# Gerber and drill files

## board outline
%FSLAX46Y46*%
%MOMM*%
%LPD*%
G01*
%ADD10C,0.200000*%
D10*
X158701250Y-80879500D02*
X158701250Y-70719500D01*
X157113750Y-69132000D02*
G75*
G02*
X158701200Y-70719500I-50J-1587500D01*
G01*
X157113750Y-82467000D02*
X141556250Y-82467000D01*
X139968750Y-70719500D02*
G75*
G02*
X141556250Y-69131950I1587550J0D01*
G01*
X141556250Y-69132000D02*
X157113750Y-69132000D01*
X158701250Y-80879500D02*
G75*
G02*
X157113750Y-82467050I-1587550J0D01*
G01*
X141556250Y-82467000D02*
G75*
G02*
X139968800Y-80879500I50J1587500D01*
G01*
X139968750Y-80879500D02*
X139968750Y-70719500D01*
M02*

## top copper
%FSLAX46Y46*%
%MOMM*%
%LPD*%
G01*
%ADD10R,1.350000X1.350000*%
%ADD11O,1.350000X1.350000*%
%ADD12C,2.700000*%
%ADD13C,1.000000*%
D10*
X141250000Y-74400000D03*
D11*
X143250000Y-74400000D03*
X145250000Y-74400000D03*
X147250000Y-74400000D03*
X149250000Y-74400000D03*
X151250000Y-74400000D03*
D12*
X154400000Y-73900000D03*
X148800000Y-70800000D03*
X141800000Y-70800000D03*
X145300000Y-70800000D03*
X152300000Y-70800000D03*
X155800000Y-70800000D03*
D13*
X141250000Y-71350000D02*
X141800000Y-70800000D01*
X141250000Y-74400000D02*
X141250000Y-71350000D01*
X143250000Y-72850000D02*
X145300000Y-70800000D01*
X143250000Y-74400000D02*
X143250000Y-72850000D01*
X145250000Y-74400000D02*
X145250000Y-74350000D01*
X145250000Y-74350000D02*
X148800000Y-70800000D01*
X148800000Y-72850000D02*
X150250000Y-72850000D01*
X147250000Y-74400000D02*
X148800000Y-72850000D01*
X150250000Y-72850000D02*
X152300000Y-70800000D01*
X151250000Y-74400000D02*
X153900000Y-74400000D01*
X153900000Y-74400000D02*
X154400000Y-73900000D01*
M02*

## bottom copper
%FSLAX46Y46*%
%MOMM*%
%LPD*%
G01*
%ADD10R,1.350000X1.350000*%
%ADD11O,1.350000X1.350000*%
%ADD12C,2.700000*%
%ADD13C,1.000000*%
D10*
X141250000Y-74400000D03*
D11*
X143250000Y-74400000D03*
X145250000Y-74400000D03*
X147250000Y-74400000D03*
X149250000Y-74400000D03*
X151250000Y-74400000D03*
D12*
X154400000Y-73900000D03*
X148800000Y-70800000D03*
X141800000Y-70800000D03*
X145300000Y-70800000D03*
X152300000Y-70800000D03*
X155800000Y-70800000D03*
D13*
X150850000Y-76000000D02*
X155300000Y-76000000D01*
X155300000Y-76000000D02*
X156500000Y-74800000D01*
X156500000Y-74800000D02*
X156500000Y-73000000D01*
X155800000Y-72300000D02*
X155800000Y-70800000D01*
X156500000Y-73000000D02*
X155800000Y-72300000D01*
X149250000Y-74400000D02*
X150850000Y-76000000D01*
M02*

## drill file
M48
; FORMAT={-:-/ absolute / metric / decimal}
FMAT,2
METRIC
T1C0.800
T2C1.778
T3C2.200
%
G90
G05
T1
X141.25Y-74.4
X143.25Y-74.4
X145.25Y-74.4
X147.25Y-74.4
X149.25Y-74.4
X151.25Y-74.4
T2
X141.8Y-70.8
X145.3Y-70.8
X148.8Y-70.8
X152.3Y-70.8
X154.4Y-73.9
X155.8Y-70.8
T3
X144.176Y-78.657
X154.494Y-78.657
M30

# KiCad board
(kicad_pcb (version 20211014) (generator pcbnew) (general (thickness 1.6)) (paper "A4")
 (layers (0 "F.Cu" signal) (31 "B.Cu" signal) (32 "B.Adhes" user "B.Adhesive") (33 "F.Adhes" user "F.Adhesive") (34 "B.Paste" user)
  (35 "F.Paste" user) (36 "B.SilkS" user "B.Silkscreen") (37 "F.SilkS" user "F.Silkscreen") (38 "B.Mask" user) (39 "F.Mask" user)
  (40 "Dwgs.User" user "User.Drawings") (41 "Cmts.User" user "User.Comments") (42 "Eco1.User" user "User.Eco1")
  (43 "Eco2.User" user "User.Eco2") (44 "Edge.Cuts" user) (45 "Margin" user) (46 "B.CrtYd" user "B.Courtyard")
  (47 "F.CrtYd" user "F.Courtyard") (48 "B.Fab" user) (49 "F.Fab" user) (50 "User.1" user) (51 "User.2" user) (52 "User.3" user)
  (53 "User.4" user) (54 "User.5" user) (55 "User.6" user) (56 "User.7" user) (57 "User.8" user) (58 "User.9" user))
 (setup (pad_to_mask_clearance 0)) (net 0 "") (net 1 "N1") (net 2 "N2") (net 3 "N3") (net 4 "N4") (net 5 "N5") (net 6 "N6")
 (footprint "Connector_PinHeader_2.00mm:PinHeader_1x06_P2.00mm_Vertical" (layer "F.Cu") (at 141.25 74.4 90)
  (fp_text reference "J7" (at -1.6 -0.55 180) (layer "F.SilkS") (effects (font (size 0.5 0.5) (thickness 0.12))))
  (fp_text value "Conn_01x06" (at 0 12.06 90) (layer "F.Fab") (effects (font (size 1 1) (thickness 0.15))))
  (pad "1" thru_hole rect (at 0 0 90) (size 1.35 1.35) (drill 0.8) (layers *.Cu *.Mask) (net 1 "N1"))
  (pad "2" thru_hole oval (at 0 2 90) (size 1.35 1.35) (drill 0.8) (layers *.Cu *.Mask) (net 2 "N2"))
  (pad "3" thru_hole oval (at 0 4 90) (size 1.35 1.35) (drill 0.8) (layers *.Cu *.Mask) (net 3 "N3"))
  (pad "4" thru_hole oval (at 0 6 90) (size 1.35 1.35) (drill 0.8) (layers *.Cu *.Mask) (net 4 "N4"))
  (pad "5" thru_hole oval (at 0 8 90) (size 1.35 1.35) (drill 0.8) (layers *.Cu *.Mask) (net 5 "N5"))
  (pad "6" thru_hole oval (at 0 10 90) (size 1.35 1.35) (drill 0.8) (layers *.Cu *.Mask) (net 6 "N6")))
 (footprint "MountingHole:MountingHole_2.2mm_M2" (layer "F.Cu") (at 154.494375 78.657)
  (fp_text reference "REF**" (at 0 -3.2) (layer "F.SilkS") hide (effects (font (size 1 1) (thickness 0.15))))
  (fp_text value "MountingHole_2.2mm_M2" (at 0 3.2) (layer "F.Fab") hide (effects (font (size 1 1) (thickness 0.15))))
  (pad "" np_thru_hole circle (at 0 0) (size 2.2 2.2) (drill 2.2) (layers *.Cu *.Mask)))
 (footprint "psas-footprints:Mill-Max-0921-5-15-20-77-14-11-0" (layer "F.Cu") (at 154.4 73.9)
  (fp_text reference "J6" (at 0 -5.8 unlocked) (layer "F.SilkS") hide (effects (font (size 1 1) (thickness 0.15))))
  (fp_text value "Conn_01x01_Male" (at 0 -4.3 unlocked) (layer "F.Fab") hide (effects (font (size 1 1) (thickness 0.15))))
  (pad "1" thru_hole circle (at 0 0) (size 2.7 2.7) (drill 1.778) (layers *.Cu *.Mask) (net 6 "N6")))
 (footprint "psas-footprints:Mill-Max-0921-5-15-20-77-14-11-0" (layer "F.Cu") (at 148.8 70.8)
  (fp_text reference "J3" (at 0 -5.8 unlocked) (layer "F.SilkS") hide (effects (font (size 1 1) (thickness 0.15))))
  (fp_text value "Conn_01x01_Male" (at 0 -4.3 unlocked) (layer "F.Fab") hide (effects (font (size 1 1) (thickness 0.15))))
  (pad "1" thru_hole circle (at 0 0) (size 2.7 2.7) (drill 1.778) (layers *.Cu *.Mask) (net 3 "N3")))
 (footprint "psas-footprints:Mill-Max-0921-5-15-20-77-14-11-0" (layer "F.Cu") (at 141.8 70.8)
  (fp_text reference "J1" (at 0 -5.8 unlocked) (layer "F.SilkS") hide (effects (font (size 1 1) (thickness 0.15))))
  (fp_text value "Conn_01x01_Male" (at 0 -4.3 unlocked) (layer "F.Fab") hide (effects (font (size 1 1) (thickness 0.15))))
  (pad "1" thru_hole circle (at 0 0) (size 2.7 2.7) (drill 1.778) (layers *.Cu *.Mask) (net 1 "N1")))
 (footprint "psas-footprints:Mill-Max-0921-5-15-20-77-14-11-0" (layer "F.Cu") (at 145.3 70.8)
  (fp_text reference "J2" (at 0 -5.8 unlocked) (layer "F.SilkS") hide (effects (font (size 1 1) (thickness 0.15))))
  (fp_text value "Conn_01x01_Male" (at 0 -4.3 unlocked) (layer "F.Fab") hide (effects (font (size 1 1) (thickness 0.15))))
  (pad "1" thru_hole circle (at 0 0) (size 2.7 2.7) (drill 1.778) (layers *.Cu *.Mask) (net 2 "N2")))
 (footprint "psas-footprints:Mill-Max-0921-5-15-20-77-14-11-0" (layer "F.Cu") (at 152.3 70.8)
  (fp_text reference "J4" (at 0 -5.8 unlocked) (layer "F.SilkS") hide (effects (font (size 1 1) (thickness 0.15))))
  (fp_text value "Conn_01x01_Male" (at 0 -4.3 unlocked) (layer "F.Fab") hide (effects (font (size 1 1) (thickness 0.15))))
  (pad "1" thru_hole circle (at 0 0) (size 2.7 2.7) (drill 1.778) (layers *.Cu *.Mask) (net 4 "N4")))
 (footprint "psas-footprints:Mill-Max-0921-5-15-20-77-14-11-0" (layer "F.Cu") (at 155.8 70.8)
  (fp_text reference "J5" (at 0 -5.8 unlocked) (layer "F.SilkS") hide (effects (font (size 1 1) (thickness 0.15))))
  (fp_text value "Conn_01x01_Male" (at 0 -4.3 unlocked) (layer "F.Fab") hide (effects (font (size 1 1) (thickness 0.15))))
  (pad "1" thru_hole circle (at 0 0) (size 2.7 2.7) (drill 1.778) (layers *.Cu *.Mask) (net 5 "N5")))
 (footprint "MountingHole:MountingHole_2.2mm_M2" (layer "F.Cu") (at 144.175625 78.657)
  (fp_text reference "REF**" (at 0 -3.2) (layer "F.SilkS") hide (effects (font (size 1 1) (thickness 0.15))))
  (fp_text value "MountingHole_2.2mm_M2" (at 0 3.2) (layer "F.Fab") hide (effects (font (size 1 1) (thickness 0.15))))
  (pad "" np_thru_hole circle (at 0 0) (size 2.2 2.2) (drill 2.2) (layers *.Cu *.Mask)))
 (gr_line (start 158.70125 80.8795) (end 158.70125 70.7195) (layer "Edge.Cuts") (width 0.2))
 (gr_arc (start 157.11375 69.132) (mid 158.236282 69.596968) (end 158.70125 70.7195) (layer "Edge.Cuts") (width 0.2))
 (gr_line (start 157.11375 82.467) (end 141.55625 82.467) (layer "Edge.Cuts") (width 0.2))
 (gr_arc (start 139.96875 70.7195) (mid 140.433718 69.596968) (end 141.55625 69.132) (layer "Edge.Cuts") (width 0.2))
 (gr_line (start 141.55625 69.132) (end 157.11375 69.132) (layer "Edge.Cuts") (width 0.2))
 (gr_arc (start 158.70125 80.8795) (mid 158.236282 82.002032) (end 157.11375 82.467) (layer "Edge.Cuts") (width 0.2))
 (gr_arc (start 141.55625 82.467) (mid 140.433718 82.002032) (end 139.96875 80.8795) (layer "Edge.Cuts") (width 0.2))
 (gr_line (start 139.96875 80.8795) (end 139.96875 70.7195) (layer "Edge.Cuts") (width 0.2))
 (segment (start 141.25 71.35) (end 141.8 70.8) (width 1) (layer "F.Cu") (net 1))
 (segment (start 141.25 74.4) (end 141.25 71.35) (width 1) (layer "F.Cu") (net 1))
 (segment (start 143.25 72.85) (end 145.3 70.8) (width 1) (layer "F.Cu") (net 2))
 (segment (start 143.25 74.4) (end 143.25 72.85) (width 1) (layer "F.Cu") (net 2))
 (segment (start 145.25 74.4) (end 145.25 74.35) (width 1) (layer "F.Cu") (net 3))
 (segment (start 145.25 74.35) (end 148.8 70.8) (width 1) (layer "F.Cu") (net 3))
 (segment (start 148.8 72.85) (end 150.25 72.85) (width 1) (layer "F.Cu") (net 4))
 (segment (start 147.25 74.4) (end 148.8 72.85) (width 1) (layer "F.Cu") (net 4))
 (segment (start 150.25 72.85) (end 152.3 70.8) (width 1) (layer "F.Cu") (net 4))
 (segment (start 150.85 76) (end 155.3 76) (width 1) (layer "B.Cu") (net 5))
 (segment (start 155.3 76) (end 156.5 74.8) (width 1) (layer "B.Cu") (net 5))
 (segment (start 156.5 74.8) (end 156.5 73) (width 1) (layer "B.Cu") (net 5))
 (segment (start 155.8 72.3) (end 155.8 70.8) (width 1) (layer "B.Cu") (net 5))
 (segment (start 156.5 73) (end 155.8 72.3) (width 1) (layer "B.Cu") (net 5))
 (segment (start 149.25 74.4) (end 150.85 76) (width 1) (layer "B.Cu") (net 5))
 (segment (start 151.25 74.4) (end 153.9 74.4) (width 1) (layer "F.Cu") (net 6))
 (segment (start 153.9 74.4) (end 154.4 73.9) (width 1) (layer "F.Cu") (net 6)))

